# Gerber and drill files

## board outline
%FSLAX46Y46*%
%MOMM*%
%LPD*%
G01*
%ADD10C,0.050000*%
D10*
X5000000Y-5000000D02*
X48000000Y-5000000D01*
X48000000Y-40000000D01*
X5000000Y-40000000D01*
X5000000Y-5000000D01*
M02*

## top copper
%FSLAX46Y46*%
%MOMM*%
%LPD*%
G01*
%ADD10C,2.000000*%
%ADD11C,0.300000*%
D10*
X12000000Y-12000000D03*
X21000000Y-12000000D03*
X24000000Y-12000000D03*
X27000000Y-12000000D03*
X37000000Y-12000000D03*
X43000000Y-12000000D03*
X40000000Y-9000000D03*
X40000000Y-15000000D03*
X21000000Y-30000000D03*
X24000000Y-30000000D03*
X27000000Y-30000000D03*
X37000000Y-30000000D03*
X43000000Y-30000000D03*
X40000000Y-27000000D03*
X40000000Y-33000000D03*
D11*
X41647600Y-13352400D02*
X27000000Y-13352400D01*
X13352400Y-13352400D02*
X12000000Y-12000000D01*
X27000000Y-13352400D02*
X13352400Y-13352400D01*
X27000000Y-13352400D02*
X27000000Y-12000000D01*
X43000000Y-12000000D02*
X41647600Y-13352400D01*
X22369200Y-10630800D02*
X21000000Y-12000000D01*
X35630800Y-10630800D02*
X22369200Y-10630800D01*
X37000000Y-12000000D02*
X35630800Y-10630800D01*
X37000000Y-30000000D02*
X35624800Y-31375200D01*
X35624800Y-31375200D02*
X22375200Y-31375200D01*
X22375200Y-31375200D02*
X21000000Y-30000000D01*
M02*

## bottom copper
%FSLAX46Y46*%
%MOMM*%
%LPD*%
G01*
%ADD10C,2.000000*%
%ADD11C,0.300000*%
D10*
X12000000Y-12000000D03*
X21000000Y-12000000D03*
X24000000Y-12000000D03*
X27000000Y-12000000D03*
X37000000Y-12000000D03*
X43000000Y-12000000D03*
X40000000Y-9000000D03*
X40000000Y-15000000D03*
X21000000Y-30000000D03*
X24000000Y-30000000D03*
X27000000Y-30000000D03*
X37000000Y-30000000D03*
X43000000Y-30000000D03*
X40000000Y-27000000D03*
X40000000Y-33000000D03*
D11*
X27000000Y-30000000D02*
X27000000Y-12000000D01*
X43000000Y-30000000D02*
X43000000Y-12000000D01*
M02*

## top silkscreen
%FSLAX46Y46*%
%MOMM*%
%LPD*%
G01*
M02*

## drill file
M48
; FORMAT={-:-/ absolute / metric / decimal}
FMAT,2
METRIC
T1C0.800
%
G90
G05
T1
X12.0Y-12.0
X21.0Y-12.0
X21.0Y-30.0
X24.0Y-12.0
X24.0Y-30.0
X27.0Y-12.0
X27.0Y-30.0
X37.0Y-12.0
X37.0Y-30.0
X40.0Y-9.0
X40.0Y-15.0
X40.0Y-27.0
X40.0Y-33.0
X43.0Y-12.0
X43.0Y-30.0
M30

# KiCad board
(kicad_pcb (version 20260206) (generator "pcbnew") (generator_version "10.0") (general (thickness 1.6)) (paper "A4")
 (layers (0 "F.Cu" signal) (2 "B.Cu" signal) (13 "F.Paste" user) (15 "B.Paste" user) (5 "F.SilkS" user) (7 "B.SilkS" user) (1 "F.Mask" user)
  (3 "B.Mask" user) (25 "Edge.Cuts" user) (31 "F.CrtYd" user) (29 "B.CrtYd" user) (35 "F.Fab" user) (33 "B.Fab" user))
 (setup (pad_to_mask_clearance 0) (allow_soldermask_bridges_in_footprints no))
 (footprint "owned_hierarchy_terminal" (layer "F.Cu") (at 12 12)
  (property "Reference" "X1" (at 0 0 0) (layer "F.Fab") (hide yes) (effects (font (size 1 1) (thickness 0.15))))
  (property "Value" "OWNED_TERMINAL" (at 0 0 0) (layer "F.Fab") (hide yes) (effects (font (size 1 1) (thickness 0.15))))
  (pad "1" thru_hole circle (at 0 0) (size 2 2) (drill 0.8) (layers "*.Cu" "*.Mask") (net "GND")))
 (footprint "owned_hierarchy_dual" (layer "F.Cu") (at 24 12)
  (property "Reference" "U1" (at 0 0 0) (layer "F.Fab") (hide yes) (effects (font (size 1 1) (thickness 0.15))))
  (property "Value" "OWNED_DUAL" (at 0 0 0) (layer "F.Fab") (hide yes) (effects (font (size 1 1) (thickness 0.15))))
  (pad "1" thru_hole circle (at -3 0) (size 2 2) (drill 0.8) (layers "*.Cu" "*.Mask") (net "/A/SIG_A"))
  (pad "2" thru_hole circle (at 0 0) (size 2 2) (drill 0.8) (layers "*.Cu" "*.Mask") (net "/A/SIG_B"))
  (pad "3" thru_hole circle (at 3 0) (size 2 2) (drill 0.8) (layers "*.Cu" "*.Mask") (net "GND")))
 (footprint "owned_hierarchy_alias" (layer "F.Cu") (at 40 12)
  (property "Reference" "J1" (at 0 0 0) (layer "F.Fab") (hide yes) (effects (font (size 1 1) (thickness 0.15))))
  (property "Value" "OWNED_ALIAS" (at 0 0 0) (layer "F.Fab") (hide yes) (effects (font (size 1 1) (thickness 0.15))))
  (pad "R" thru_hole circle (at -3 0) (size 2 2) (drill 0.8) (layers "*.Cu" "*.Mask") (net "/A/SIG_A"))
  (pad "T" thru_hole circle (at 3 0) (size 2 2) (drill 0.8) (layers "*.Cu" "*.Mask") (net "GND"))
  (pad "MP" thru_hole circle (at 0 -3) (size 2 2) (drill 0.8) (layers "*.Cu" "*.Mask"))
  (pad "MP" thru_hole circle (at 0 3) (size 2 2) (drill 0.8) (layers "*.Cu" "*.Mask")))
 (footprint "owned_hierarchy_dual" (layer "F.Cu") (at 24 30)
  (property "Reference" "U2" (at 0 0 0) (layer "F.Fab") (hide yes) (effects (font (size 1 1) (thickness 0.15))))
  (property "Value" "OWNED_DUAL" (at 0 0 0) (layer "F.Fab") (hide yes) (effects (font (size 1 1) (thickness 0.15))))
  (pad "1" thru_hole circle (at -3 0) (size 2 2) (drill 0.8) (layers "*.Cu" "*.Mask") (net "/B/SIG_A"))
  (pad "2" thru_hole circle (at 0 0) (size 2 2) (drill 0.8) (layers "*.Cu" "*.Mask") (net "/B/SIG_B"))
  (pad "3" thru_hole circle (at 3 0) (size 2 2) (drill 0.8) (layers "*.Cu" "*.Mask") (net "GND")))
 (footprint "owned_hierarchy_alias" (layer "F.Cu") (at 40 30)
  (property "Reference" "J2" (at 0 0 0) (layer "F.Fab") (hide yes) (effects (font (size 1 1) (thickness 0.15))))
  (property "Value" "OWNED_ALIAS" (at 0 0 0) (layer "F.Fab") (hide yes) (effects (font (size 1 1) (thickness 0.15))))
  (pad "R" thru_hole circle (at -3 0) (size 2 2) (drill 0.8) (layers "*.Cu" "*.Mask") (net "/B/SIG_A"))
  (pad "T" thru_hole circle (at 3 0) (size 2 2) (drill 0.8) (layers "*.Cu" "*.Mask") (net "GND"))
  (pad "MP" thru_hole circle (at 0 -3) (size 2 2) (drill 0.8) (layers "*.Cu" "*.Mask"))
  (pad "MP" thru_hole circle (at 0 3) (size 2 2) (drill 0.8) (layers "*.Cu" "*.Mask")))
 (gr_rect (start 5 5) (end 48 40) (stroke (width 0.05) (type default)) (fill none) (layer "Edge.Cuts"))
 (segment (start 41.6476 13.3524) (end 27 13.3524) (width 0.3) (layer "F.Cu") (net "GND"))
 (segment (start 13.3524 13.3524) (end 12 12) (width 0.3) (layer "F.Cu") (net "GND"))
 (segment (start 27 13.3524) (end 13.3524 13.3524) (width 0.3) (layer "F.Cu") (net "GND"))
 (segment (start 27 13.3524) (end 27 12) (width 0.3) (layer "F.Cu") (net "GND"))
 (segment (start 43 12) (end 41.6476 13.3524) (width 0.3) (layer "F.Cu") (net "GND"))
 (segment (start 27 30) (end 27 12) (width 0.3) (layer "B.Cu") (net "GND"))
 (segment (start 43 30) (end 43 12) (width 0.3) (layer "B.Cu") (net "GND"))
 (segment (start 22.3692 10.6308) (end 21 12) (width 0.3) (layer "F.Cu") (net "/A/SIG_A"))
 (segment (start 35.6308 10.6308) (end 22.3692 10.6308) (width 0.3) (layer "F.Cu") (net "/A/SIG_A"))
 (segment (start 37 12) (end 35.6308 10.6308) (width 0.3) (layer "F.Cu") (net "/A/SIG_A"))
 (segment (start 37 30) (end 35.6248 31.3752) (width 0.3) (layer "F.Cu") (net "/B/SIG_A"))
 (segment (start 35.6248 31.3752) (end 22.3752 31.3752) (width 0.3) (layer "F.Cu") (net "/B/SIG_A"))
 (segment (start 22.3752 31.3752) (end 21 30) (width 0.3) (layer "F.Cu") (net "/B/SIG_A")))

